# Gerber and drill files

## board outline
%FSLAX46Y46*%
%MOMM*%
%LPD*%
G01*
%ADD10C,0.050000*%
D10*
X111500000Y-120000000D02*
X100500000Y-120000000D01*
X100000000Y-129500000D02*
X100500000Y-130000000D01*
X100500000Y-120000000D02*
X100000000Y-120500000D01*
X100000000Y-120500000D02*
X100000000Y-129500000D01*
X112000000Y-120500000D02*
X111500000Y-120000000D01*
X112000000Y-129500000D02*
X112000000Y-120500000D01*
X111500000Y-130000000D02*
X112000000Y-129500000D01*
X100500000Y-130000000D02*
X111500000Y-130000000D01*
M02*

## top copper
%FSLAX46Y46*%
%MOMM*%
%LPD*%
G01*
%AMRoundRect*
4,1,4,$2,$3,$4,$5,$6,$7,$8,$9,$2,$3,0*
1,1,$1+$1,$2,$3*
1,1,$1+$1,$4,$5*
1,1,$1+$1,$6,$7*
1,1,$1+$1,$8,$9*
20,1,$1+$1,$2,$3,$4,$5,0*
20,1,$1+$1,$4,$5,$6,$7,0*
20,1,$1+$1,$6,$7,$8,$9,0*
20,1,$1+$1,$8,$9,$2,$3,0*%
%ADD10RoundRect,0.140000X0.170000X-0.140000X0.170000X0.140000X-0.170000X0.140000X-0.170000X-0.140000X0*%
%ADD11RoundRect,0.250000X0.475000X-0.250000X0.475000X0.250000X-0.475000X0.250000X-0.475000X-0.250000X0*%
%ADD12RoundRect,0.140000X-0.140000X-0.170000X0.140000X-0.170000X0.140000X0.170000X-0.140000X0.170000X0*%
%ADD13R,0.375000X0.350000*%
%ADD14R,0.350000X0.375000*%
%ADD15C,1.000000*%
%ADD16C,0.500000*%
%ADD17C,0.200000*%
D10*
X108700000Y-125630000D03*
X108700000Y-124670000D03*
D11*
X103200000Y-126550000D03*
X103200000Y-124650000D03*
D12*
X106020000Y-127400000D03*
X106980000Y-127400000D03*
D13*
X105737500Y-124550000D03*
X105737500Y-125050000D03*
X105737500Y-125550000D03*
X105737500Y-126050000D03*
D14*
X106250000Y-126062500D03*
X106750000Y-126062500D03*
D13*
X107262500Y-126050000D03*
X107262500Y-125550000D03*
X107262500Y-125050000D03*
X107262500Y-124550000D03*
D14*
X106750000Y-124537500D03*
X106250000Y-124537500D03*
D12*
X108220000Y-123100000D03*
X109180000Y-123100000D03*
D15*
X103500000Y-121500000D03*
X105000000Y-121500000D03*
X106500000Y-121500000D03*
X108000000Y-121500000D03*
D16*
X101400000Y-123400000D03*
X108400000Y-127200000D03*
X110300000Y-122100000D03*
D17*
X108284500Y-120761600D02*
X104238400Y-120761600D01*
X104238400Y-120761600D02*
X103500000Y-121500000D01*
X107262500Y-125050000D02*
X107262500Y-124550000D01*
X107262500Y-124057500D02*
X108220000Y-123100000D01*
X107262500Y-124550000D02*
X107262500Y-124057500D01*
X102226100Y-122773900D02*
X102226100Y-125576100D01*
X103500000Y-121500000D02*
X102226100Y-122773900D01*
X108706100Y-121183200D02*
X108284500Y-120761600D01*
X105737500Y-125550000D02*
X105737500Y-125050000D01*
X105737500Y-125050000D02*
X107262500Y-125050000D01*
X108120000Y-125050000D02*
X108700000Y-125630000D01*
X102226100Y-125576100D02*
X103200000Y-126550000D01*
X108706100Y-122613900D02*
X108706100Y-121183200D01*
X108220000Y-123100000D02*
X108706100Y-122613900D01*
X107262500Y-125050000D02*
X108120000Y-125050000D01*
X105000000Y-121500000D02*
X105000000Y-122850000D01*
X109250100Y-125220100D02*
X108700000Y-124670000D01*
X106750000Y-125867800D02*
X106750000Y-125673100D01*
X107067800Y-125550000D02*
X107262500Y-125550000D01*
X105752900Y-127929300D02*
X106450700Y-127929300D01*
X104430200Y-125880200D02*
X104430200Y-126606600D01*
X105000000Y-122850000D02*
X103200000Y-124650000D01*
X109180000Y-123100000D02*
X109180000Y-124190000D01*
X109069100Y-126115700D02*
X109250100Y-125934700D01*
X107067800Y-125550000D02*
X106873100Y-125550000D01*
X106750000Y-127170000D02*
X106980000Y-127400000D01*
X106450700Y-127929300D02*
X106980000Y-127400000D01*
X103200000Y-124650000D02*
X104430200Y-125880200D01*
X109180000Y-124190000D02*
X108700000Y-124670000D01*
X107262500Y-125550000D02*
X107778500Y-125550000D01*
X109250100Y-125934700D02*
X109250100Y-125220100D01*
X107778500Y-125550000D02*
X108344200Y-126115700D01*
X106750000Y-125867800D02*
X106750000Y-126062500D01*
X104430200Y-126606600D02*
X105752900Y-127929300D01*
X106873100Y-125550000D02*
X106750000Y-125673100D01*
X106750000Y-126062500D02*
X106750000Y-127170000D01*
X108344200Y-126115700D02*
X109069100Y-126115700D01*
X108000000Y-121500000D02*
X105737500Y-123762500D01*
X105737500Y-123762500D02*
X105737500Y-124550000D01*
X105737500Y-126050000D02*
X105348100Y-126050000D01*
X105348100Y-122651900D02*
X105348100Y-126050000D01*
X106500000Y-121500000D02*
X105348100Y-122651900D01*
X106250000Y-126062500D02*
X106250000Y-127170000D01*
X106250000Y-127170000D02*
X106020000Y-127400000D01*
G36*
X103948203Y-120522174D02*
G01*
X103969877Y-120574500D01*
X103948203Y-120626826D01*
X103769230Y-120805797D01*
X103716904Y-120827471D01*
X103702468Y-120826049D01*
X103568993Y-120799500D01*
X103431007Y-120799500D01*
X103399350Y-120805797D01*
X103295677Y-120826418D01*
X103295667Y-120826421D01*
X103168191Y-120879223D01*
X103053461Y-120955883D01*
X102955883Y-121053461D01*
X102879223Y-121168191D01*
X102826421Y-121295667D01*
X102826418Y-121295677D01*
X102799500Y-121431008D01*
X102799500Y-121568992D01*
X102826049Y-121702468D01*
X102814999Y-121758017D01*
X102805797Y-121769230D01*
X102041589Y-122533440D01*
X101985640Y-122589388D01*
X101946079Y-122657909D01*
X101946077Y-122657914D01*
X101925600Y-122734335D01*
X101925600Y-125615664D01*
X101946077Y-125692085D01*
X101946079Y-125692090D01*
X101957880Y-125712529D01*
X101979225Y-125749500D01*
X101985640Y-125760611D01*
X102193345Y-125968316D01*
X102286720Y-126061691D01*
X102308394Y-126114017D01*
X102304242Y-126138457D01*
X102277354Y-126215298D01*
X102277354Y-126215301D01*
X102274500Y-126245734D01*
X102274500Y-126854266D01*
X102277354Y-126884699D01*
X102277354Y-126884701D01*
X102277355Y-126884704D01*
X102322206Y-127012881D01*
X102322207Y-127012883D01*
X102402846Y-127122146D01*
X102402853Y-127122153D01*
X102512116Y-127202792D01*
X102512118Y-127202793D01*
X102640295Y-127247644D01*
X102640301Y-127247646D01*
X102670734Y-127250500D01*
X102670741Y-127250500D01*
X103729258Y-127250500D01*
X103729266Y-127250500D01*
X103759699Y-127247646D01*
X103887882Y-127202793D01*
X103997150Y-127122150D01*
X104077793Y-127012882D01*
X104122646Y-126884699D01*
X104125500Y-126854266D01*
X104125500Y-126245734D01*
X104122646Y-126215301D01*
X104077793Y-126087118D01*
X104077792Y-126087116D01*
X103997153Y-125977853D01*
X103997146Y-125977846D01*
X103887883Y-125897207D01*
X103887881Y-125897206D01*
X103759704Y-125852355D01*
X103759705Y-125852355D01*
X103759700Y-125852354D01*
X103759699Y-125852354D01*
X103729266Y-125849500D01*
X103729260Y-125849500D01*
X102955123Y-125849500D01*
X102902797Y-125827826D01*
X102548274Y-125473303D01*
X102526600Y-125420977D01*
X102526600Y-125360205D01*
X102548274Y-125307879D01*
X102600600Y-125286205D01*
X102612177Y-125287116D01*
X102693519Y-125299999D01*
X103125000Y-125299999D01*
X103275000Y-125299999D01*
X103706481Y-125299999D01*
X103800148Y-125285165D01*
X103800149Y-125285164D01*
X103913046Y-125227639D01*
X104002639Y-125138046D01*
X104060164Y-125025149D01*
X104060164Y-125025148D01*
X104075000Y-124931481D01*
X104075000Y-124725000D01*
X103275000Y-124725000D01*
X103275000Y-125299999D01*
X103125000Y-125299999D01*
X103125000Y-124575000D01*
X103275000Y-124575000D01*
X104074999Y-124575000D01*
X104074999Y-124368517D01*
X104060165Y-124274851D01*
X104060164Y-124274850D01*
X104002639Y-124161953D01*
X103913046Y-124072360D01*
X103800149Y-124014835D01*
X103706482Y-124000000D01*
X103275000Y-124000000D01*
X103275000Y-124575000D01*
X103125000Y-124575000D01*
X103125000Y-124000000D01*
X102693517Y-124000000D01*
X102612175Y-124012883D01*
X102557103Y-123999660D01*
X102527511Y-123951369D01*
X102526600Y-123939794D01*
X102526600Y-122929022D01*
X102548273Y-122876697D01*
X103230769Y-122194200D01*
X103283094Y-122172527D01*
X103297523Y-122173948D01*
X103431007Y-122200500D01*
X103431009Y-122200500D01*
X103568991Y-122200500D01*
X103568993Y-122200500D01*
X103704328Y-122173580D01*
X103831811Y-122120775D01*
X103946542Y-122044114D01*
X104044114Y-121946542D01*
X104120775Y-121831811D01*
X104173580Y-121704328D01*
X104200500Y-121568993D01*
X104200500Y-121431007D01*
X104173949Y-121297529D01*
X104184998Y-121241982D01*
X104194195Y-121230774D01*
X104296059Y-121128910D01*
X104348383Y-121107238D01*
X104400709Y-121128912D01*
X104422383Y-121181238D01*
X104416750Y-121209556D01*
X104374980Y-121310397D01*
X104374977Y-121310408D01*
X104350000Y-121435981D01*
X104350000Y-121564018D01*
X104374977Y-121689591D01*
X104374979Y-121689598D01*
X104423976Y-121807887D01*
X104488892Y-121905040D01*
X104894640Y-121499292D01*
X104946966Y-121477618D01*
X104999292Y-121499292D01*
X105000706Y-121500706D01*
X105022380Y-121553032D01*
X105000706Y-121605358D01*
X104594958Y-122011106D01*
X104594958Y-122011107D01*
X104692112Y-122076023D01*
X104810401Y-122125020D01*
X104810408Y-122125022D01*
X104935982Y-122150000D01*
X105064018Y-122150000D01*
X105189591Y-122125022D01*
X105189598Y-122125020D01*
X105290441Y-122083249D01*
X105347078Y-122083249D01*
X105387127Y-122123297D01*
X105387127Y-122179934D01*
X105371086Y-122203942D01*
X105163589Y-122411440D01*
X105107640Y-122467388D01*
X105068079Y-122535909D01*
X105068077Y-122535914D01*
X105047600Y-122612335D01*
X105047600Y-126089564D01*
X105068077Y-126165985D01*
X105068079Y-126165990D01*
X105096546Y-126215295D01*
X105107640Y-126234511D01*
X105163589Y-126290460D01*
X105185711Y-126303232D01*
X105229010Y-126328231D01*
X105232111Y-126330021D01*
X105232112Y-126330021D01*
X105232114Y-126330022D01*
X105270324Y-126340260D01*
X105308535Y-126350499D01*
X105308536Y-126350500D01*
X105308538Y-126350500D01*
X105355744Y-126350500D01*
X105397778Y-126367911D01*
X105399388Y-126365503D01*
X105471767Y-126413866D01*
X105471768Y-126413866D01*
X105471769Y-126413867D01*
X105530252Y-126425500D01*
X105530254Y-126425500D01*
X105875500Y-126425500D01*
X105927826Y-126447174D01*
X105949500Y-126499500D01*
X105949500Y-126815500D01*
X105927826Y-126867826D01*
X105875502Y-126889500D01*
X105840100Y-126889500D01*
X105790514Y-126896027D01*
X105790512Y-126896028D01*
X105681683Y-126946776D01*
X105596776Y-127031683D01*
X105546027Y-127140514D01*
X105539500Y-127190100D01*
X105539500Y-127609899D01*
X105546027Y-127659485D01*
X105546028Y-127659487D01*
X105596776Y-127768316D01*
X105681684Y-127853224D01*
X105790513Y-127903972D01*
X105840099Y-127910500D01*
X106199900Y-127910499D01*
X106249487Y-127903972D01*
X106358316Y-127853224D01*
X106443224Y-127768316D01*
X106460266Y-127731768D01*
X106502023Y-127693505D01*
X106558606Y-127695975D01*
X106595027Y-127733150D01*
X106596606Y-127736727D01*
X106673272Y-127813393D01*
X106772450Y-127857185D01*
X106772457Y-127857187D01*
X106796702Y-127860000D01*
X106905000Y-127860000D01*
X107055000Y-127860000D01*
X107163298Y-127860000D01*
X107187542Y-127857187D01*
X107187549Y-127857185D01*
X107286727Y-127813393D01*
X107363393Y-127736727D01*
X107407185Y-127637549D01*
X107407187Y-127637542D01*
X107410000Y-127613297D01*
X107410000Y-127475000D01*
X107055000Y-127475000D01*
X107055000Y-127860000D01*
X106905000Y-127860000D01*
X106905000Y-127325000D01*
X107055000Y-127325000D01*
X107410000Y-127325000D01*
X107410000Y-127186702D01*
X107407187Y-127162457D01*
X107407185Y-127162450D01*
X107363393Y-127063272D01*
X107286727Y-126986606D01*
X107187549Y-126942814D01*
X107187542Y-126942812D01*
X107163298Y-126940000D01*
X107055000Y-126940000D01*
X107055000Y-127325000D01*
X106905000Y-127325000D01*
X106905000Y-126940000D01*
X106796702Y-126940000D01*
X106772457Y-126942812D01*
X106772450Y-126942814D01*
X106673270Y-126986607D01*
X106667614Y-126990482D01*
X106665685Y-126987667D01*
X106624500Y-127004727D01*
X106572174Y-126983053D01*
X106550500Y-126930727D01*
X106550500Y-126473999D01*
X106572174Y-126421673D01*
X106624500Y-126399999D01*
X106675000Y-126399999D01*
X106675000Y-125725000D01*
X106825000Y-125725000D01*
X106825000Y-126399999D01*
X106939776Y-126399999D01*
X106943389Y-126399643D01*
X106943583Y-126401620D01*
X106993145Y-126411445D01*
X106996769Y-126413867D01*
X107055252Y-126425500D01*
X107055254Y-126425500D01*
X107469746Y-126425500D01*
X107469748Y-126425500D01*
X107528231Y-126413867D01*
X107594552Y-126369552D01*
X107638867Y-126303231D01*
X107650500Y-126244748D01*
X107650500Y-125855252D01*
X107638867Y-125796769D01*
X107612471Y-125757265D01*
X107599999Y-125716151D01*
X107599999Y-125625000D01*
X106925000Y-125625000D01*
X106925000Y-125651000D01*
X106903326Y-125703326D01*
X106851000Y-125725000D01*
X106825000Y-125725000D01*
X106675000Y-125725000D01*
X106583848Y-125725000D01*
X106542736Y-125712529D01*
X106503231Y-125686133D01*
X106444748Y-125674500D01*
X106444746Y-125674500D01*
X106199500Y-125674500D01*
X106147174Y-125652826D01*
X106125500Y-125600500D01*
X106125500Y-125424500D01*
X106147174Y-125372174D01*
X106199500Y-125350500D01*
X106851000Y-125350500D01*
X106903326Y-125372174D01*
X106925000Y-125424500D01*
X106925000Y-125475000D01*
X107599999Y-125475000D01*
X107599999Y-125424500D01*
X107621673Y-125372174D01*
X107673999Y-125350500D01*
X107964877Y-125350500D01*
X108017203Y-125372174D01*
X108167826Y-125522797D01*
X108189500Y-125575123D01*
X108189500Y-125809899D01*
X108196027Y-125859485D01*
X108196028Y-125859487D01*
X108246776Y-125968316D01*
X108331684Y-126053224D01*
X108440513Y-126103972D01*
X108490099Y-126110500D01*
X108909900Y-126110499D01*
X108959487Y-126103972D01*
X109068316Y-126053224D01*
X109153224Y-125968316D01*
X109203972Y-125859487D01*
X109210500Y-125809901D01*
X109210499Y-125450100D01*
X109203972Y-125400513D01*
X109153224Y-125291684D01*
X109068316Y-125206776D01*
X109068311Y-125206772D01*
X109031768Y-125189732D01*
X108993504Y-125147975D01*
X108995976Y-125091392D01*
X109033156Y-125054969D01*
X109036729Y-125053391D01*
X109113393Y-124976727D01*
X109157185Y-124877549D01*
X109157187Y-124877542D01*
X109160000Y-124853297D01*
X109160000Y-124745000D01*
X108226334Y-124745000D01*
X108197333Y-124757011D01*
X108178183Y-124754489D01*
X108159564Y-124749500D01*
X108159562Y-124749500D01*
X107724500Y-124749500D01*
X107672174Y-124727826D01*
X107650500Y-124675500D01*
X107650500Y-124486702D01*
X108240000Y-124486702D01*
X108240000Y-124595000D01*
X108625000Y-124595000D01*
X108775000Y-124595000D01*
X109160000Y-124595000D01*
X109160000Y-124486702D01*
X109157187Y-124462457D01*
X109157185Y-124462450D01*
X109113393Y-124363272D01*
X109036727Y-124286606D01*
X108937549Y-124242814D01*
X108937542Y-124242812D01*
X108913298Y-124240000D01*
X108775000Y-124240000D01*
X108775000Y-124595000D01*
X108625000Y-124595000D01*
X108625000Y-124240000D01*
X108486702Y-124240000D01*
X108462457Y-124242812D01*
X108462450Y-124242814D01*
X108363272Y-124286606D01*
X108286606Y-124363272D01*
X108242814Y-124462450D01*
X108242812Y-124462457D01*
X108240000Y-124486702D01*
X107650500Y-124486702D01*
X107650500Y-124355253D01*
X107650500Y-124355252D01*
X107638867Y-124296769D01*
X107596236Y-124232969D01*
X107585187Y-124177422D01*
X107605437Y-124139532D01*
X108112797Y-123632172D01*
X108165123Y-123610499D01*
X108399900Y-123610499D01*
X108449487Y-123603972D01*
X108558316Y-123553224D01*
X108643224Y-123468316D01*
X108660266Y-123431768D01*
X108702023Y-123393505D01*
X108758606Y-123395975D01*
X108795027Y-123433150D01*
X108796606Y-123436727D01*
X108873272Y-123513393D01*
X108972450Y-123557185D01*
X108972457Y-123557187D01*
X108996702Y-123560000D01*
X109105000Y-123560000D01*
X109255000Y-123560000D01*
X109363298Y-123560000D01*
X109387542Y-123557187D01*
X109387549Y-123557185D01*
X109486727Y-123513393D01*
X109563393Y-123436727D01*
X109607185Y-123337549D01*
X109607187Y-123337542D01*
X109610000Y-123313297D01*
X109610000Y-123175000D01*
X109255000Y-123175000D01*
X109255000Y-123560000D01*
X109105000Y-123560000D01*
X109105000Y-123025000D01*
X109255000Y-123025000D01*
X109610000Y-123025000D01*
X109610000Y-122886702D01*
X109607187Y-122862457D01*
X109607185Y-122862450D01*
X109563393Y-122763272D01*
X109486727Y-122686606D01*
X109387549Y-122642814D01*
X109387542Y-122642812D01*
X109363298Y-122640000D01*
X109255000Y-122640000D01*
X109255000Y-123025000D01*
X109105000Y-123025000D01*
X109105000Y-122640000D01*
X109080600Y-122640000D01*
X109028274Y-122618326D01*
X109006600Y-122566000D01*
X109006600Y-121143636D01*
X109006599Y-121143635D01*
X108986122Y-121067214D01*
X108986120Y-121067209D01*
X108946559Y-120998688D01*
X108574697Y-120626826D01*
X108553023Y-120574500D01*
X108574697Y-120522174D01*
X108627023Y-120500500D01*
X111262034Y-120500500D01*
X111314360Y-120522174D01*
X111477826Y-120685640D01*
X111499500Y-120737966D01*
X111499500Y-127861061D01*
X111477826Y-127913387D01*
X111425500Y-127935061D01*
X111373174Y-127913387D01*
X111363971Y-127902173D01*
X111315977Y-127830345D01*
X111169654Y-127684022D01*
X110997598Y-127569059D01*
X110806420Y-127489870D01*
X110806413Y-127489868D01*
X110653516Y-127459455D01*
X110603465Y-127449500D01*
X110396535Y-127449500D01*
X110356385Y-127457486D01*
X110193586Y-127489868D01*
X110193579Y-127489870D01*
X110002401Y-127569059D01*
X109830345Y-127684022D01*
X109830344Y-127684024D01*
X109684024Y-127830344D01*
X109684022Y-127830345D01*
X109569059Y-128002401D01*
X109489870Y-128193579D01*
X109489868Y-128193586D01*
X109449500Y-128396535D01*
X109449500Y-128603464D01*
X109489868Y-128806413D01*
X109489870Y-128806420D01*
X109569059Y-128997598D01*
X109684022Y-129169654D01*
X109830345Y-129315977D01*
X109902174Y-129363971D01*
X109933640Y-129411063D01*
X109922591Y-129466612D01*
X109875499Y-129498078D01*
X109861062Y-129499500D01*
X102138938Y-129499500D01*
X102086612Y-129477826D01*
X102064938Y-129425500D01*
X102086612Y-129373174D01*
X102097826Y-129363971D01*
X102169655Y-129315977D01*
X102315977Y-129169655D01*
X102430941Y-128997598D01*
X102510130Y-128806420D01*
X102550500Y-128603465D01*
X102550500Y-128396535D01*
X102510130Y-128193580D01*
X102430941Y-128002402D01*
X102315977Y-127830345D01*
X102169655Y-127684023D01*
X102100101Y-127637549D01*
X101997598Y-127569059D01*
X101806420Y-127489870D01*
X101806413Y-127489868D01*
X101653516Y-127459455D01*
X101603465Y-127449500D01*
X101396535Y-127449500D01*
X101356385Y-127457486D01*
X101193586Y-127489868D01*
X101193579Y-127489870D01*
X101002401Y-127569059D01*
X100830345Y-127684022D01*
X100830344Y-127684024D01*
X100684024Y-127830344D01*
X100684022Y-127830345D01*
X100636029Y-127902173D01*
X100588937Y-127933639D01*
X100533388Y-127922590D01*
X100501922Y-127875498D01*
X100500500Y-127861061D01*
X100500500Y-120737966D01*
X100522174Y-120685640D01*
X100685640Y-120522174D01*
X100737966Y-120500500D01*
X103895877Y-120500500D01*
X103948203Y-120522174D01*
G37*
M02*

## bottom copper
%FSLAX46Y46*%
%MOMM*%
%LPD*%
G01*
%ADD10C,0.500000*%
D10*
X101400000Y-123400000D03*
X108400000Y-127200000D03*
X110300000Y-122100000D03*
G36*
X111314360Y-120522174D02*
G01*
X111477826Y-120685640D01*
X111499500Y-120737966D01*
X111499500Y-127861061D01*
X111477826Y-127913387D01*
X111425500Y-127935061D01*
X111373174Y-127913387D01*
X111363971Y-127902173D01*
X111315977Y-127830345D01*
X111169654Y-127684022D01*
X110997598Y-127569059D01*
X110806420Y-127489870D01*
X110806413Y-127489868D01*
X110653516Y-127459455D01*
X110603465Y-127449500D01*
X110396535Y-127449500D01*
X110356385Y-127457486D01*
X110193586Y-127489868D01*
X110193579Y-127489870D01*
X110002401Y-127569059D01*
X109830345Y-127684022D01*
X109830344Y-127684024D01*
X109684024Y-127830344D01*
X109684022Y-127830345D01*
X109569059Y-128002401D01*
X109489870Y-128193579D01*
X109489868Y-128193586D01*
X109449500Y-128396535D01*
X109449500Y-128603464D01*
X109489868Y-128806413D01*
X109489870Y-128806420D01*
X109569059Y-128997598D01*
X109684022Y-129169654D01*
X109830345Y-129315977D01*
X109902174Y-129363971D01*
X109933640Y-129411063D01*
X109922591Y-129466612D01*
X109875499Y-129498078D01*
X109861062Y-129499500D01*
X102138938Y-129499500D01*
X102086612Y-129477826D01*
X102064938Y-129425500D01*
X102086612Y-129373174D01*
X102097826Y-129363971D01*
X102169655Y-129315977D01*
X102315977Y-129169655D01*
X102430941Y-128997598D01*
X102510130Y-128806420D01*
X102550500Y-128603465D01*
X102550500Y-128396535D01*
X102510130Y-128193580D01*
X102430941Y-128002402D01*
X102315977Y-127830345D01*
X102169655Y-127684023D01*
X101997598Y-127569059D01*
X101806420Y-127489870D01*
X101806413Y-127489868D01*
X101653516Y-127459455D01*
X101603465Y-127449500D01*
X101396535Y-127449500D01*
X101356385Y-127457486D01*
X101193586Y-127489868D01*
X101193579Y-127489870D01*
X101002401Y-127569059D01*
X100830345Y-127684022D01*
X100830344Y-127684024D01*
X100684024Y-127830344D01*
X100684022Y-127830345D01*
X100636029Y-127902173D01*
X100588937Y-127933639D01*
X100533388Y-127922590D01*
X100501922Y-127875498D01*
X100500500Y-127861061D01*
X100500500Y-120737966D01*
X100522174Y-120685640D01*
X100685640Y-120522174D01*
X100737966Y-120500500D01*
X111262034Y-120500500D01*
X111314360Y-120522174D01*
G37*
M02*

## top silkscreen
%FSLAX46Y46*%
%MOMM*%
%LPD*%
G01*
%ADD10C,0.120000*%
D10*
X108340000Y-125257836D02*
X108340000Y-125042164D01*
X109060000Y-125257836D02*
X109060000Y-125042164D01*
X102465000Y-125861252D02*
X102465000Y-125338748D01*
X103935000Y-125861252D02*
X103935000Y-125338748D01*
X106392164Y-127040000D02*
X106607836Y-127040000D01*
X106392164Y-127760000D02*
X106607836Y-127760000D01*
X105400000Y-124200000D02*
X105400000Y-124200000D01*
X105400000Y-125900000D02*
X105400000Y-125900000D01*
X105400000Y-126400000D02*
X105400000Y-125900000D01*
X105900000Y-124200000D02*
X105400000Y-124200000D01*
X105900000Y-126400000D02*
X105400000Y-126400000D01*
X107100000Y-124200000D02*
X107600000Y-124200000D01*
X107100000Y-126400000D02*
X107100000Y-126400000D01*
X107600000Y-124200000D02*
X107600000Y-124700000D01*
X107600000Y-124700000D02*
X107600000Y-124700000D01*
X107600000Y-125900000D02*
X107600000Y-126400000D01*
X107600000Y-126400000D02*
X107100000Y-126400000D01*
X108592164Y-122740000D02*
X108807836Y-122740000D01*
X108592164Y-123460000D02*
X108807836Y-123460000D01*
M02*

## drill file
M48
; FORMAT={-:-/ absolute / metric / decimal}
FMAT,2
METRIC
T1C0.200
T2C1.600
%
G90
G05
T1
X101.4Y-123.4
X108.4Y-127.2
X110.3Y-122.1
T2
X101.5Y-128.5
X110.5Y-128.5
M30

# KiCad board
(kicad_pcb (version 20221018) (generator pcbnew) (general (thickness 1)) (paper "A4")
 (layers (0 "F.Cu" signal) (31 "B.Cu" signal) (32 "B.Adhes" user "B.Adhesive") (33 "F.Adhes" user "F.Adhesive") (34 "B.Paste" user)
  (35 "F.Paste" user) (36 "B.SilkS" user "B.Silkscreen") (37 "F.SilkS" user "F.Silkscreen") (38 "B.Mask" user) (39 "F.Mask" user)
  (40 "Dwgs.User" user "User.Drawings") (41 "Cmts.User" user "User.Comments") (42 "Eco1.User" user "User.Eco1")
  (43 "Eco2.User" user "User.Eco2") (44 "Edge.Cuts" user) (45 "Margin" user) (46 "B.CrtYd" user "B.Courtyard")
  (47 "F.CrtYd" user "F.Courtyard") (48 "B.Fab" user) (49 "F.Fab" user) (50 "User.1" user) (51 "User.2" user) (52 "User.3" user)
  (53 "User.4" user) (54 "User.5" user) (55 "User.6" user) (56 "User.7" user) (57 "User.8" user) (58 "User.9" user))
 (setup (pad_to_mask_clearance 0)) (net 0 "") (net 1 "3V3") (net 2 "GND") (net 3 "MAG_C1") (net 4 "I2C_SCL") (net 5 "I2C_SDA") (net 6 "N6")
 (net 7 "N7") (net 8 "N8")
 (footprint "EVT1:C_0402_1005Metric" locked (layer "F.Cu") (at 108.7 125.15 90)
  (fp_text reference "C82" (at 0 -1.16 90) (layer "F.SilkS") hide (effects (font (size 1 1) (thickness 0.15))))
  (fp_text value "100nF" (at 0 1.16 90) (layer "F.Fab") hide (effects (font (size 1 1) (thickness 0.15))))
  (fp_line (start -0.107836 -0.36) (end 0.107836 -0.36) (stroke (width 0.12) (type solid)) (layer "F.SilkS"))
  (fp_line (start -0.107836 0.36) (end 0.107836 0.36) (stroke (width 0.12) (type solid)) (layer "F.SilkS"))
  (pad "1" smd roundrect locked (at -0.48 0 90) (size 0.56 0.62) (layers "F.Cu" "F.Paste" "F.Mask") (roundrect_rratio 0.25) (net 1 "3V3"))
  (pad "2" smd roundrect locked (at 0.48 0 90) (size 0.56 0.62) (layers "F.Cu" "F.Paste" "F.Mask") (roundrect_rratio 0.25) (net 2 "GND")))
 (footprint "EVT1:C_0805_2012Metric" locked (layer "F.Cu") (at 103.2 125.6 90)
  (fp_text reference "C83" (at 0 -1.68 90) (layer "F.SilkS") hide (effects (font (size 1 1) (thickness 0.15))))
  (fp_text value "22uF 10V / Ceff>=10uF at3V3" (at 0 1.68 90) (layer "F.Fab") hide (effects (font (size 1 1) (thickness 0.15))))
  (fp_line (start -0.261252 -0.735) (end 0.261252 -0.735) (stroke (width 0.12) (type solid)) (layer "F.SilkS"))
  (fp_line (start -0.261252 0.735) (end 0.261252 0.735) (stroke (width 0.12) (type solid)) (layer "F.SilkS"))
  (pad "1" smd roundrect locked (at -0.95 0 90) (size 1 1.45) (layers "F.Cu" "F.Paste" "F.Mask") (roundrect_rratio 0.25) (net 1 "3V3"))
  (pad "2" smd roundrect locked (at 0.95 0 90) (size 1 1.45) (layers "F.Cu" "F.Paste" "F.Mask") (roundrect_rratio 0.25) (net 2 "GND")))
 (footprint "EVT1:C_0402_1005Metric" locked (layer "F.Cu") (at 106.5 127.4)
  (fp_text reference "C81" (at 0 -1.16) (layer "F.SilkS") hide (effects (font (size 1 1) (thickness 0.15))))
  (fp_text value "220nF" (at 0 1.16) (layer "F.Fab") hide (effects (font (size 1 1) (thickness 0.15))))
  (fp_line (start -0.107836 -0.36) (end 0.107836 -0.36) (stroke (width 0.12) (type solid)) (layer "F.SilkS"))
  (fp_line (start -0.107836 0.36) (end 0.107836 0.36) (stroke (width 0.12) (type solid)) (layer "F.SilkS"))
  (pad "1" smd roundrect locked (at -0.48 0) (size 0.56 0.62) (layers "F.Cu" "F.Paste" "F.Mask") (roundrect_rratio 0.25) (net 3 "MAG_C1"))
  (pad "2" smd roundrect locked (at 0.48 0) (size 0.56 0.62) (layers "F.Cu" "F.Paste" "F.Mask") (roundrect_rratio 0.25) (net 2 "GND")))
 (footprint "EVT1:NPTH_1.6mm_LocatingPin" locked (layer "F.Cu") (at 101.5 128.5)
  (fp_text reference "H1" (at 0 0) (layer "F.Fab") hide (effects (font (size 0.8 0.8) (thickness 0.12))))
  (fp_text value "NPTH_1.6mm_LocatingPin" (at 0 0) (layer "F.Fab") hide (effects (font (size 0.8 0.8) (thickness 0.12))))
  (pad "" np_thru_hole circle locked (at 0 0) (size 1.6 1.6) (drill 1.6) (layers "*.Cu" "*.Mask")))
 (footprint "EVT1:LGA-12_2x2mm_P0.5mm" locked (layer "F.Cu") (at 106.5 125.3)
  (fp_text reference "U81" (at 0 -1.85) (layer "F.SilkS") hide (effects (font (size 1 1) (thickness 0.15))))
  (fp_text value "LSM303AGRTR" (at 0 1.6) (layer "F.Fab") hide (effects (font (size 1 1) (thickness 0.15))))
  (fp_line (start -1.1 -1.1) (end -1.1 -1.1) (stroke (width 0.12) (type solid)) (layer "F.SilkS"))
  (fp_line (start -1.1 0.6) (end -1.1 0.6) (stroke (width 0.12) (type solid)) (layer "F.SilkS"))
  (fp_line (start -1.1 1.1) (end -1.1 0.6) (stroke (width 0.12) (type solid)) (layer "F.SilkS"))
  (fp_line (start -0.6 -1.1) (end -1.1 -1.1) (stroke (width 0.12) (type solid)) (layer "F.SilkS"))
  (fp_line (start -0.6 1.1) (end -1.1 1.1) (stroke (width 0.12) (type solid)) (layer "F.SilkS"))
  (fp_line (start 0.6 -1.1) (end 1.1 -1.1) (stroke (width 0.12) (type solid)) (layer "F.SilkS"))
  (fp_line (start 0.6 1.1) (end 0.6 1.1) (stroke (width 0.12) (type solid)) (layer "F.SilkS"))
  (fp_line (start 1.1 -1.1) (end 1.1 -0.6) (stroke (width 0.12) (type solid)) (layer "F.SilkS"))
  (fp_line (start 1.1 -0.6) (end 1.1 -0.6) (stroke (width 0.12) (type solid)) (layer "F.SilkS"))
  (fp_line (start 1.1 0.6) (end 1.1 1.1) (stroke (width 0.12) (type solid)) (layer "F.SilkS"))
  (fp_line (start 1.1 1.1) (end 0.6 1.1) (stroke (width 0.12) (type solid)) (layer "F.SilkS"))
  (pad "1" smd rect locked (at -0.7625 -0.75) (size 0.375 0.35) (layers "F.Cu" "F.Paste" "F.Mask") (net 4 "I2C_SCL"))
  (pad "2" smd rect locked (at -0.7625 -0.25) (size 0.375 0.35) (layers "F.Cu" "F.Paste" "F.Mask") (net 1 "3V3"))
  (pad "3" smd rect locked (at -0.7625 0.25) (size 0.375 0.35) (layers "F.Cu" "F.Paste" "F.Mask") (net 1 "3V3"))
  (pad "4" smd rect locked (at -0.7625 0.75) (size 0.375 0.35) (layers "F.Cu" "F.Paste" "F.Mask") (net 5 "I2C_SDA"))
  (pad "5" smd rect locked (at -0.25 0.7625 90) (size 0.375 0.35) (layers "F.Cu" "F.Paste" "F.Mask") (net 3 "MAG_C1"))
  (pad "6" smd rect locked (at 0.25 0.7625 90) (size 0.375 0.35) (layers "F.Cu" "F.Paste" "F.Mask") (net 2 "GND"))
  (pad "7" smd rect locked (at 0.7625 0.75) (size 0.375 0.35) (layers "F.Cu" "F.Paste" "F.Mask") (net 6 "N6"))
  (pad "8" smd rect locked (at 0.7625 0.25) (size 0.375 0.35) (layers "F.Cu" "F.Paste" "F.Mask") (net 2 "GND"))
  (pad "9" smd rect locked (at 0.7625 -0.25) (size 0.375 0.35) (layers "F.Cu" "F.Paste" "F.Mask") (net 1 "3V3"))
  (pad "10" smd rect locked (at 0.7625 -0.75) (size 0.375 0.35) (layers "F.Cu" "F.Paste" "F.Mask") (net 1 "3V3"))
  (pad "11" smd rect locked (at 0.25 -0.7625 90) (size 0.375 0.35) (layers "F.Cu" "F.Paste" "F.Mask") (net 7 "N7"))
  (pad "12" smd rect locked (at -0.25 -0.7625 90) (size 0.375 0.35) (layers "F.Cu" "F.Paste" "F.Mask") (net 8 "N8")))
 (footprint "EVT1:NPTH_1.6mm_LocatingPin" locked (layer "F.Cu") (at 110.5 128.5)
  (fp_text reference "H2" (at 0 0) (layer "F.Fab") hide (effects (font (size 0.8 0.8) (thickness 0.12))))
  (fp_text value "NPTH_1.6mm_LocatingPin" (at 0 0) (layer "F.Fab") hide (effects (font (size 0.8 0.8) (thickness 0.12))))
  (pad "" np_thru_hole circle locked (at 0 0) (size 1.6 1.6) (drill 1.6) (layers "*.Cu" "*.Mask")))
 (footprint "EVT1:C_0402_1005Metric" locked (layer "F.Cu") (at 108.7 123.1)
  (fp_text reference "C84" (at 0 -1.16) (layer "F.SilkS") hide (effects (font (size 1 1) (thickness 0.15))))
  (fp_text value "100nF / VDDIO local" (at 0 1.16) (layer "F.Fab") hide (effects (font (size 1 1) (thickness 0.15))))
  (fp_line (start -0.107836 -0.36) (end 0.107836 -0.36) (stroke (width 0.12) (type solid)) (layer "F.SilkS"))
  (fp_line (start -0.107836 0.36) (end 0.107836 0.36) (stroke (width 0.12) (type solid)) (layer "F.SilkS"))
  (pad "1" smd roundrect locked (at -0.48 0) (size 0.56 0.62) (layers "F.Cu" "F.Paste" "F.Mask") (roundrect_rratio 0.25) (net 1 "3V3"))
  (pad "2" smd roundrect locked (at 0.48 0) (size 0.56 0.62) (layers "F.Cu" "F.Paste" "F.Mask") (roundrect_rratio 0.25) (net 2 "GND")))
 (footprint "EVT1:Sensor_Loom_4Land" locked (layer "F.Cu") (at 103.5 121.5)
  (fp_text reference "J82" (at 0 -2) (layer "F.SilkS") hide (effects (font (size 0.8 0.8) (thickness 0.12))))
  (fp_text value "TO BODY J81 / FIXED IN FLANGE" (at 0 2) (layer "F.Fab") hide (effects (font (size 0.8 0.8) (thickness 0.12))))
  (pad "1" smd circle locked (at 0 0) (size 1 1) (layers "F.Cu" "F.Paste" "F.Mask") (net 1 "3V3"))
  (pad "2" smd circle locked (at 1.5 0) (size 1 1) (layers "F.Cu" "F.Paste" "F.Mask") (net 2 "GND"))
  (pad "3" smd circle locked (at 3 0) (size 1 1) (layers "F.Cu" "F.Paste" "F.Mask") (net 5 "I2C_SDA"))
  (pad "4" smd circle locked (at 4.5 0) (size 1 1) (layers "F.Cu" "F.Paste" "F.Mask") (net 4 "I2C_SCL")))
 (gr_line (start 111.5 120) (end 100.5 120) (stroke (width 0.05) (type default)) (layer "Edge.Cuts"))
 (gr_line (start 100 129.5) (end 100.5 130) (stroke (width 0.05) (type default)) (layer "Edge.Cuts"))
 (gr_line (start 100.5 120) (end 100 120.5) (stroke (width 0.05) (type default)) (layer "Edge.Cuts"))
 (gr_line (start 100 120.5) (end 100 129.5) (stroke (width 0.05) (type default)) (layer "Edge.Cuts"))
 (gr_line (start 112 120.5) (end 111.5 120) (stroke (width 0.05) (type default)) (layer "Edge.Cuts"))
 (gr_line (start 112 129.5) (end 112 120.5) (stroke (width 0.05) (type default)) (layer "Edge.Cuts"))
 (gr_line (start 111.5 130) (end 112 129.5) (stroke (width 0.05) (type default)) (layer "Edge.Cuts"))
 (gr_line (start 100.5 130) (end 111.5 130) (stroke (width 0.05) (type default)) (layer "Edge.Cuts"))
 (segment (start 108.2845 120.7616) (end 104.2384 120.7616) (width 0.2) (layer "F.Cu") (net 1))
 (segment (start 104.2384 120.7616) (end 103.5 121.5) (width 0.2) (layer "F.Cu") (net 1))
 (segment (start 107.2625 125.05) (end 107.2625 124.55) (width 0.2) (layer "F.Cu") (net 1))
 (segment (start 107.2625 124.0575) (end 108.22 123.1) (width 0.2) (layer "F.Cu") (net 1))
 (segment (start 107.2625 124.55) (end 107.2625 124.0575) (width 0.2) (layer "F.Cu") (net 1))
 (segment (start 102.2261 122.7739) (end 102.2261 125.5761) (width 0.2) (layer "F.Cu") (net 1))
 (segment (start 103.5 121.5) (end 102.2261 122.7739) (width 0.2) (layer "F.Cu") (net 1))
 (segment (start 108.7061 121.1832) (end 108.2845 120.7616) (width 0.2) (layer "F.Cu") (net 1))
 (segment (start 105.7375 125.55) (end 105.7375 125.05) (width 0.2) (layer "F.Cu") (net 1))
 (segment (start 105.7375 125.05) (end 107.2625 125.05) (width 0.2) (layer "F.Cu") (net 1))
 (segment (start 108.12 125.05) (end 108.7 125.63) (width 0.2) (layer "F.Cu") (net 1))
 (segment (start 102.2261 125.5761) (end 103.2 126.55) (width 0.2) (layer "F.Cu") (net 1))
 (segment (start 108.7061 122.6139) (end 108.7061 121.1832) (width 0.2) (layer "F.Cu") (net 1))
 (segment (start 108.22 123.1) (end 108.7061 122.6139) (width 0.2) (layer "F.Cu") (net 1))
 (segment (start 107.2625 125.05) (end 108.12 125.05) (width 0.2) (layer "F.Cu") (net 1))
 (segment (start 105 121.5) (end 105 122.85) (width 0.2) (layer "F.Cu") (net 2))
 (segment (start 109.2501 125.2201) (end 108.7 124.67) (width 0.2) (layer "F.Cu") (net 2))
 (segment (start 106.75 125.8678) (end 106.75 125.6731) (width 0.2) (layer "F.Cu") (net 2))
 (segment (start 107.0678 125.55) (end 107.2625 125.55) (width 0.2) (layer "F.Cu") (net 2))
 (segment (start 105.7529 127.9293) (end 106.4507 127.9293) (width 0.2) (layer "F.Cu") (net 2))
 (segment (start 104.4302 125.8802) (end 104.4302 126.6066) (width 0.2) (layer "F.Cu") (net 2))
 (segment (start 105 122.85) (end 103.2 124.65) (width 0.2) (layer "F.Cu") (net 2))
 (segment (start 109.18 123.1) (end 109.18 124.19) (width 0.2) (layer "F.Cu") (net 2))
 (segment (start 109.0691 126.1157) (end 109.2501 125.9347) (width 0.2) (layer "F.Cu") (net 2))
 (segment (start 107.0678 125.55) (end 106.8731 125.55) (width 0.2) (layer "F.Cu") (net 2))
 (segment (start 106.75 127.17) (end 106.98 127.4) (width 0.2) (layer "F.Cu") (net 2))
 (segment (start 106.4507 127.9293) (end 106.98 127.4) (width 0.2) (layer "F.Cu") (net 2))
 (segment (start 103.2 124.65) (end 104.4302 125.8802) (width 0.2) (layer "F.Cu") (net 2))
 (segment (start 109.18 124.19) (end 108.7 124.67) (width 0.2) (layer "F.Cu") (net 2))
 (segment (start 107.2625 125.55) (end 107.7785 125.55) (width 0.2) (layer "F.Cu") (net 2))
 (segment (start 109.2501 125.9347) (end 109.2501 125.2201) (width 0.2) (layer "F.Cu") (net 2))
 (segment (start 107.7785 125.55) (end 108.3442 126.1157) (width 0.2) (layer "F.Cu") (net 2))
 (segment (start 106.75 125.8678) (end 106.75 126.0625) (width 0.2) (layer "F.Cu") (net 2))
 (segment (start 104.4302 126.6066) (end 105.7529 127.9293) (width 0.2) (layer "F.Cu") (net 2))
 (segment (start 106.8731 125.55) (end 106.75 125.6731) (width 0.2) (layer "F.Cu") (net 2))
 (segment (start 106.75 126.0625) (end 106.75 127.17) (width 0.2) (layer "F.Cu") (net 2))
 (segment (start 108.3442 126.1157) (end 109.0691 126.1157) (width 0.2) (layer "F.Cu") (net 2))
 (via (at 101.4 123.4) (size 0.5) (drill 0.2) (layers "F.Cu" "B.Cu") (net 2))
 (via (at 108.4 127.2) (size 0.5) (drill 0.2) (layers "F.Cu" "B.Cu") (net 2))
 (via (at 110.3 122.1) (size 0.5) (drill 0.2) (layers "F.Cu" "B.Cu") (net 2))
 (segment (start 108 121.5) (end 105.7375 123.7625) (width 0.2) (layer "F.Cu") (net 4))
 (segment (start 105.7375 123.7625) (end 105.7375 124.55) (width 0.2) (layer "F.Cu") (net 4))
 (segment (start 105.7375 126.05) (end 105.3481 126.05) (width 0.2) (layer "F.Cu") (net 5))
 (segment (start 105.3481 122.6519) (end 105.3481 126.05) (width 0.2) (layer "F.Cu") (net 5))
 (segment (start 106.5 121.5) (end 105.3481 122.6519) (width 0.2) (layer "F.Cu") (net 5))
 (segment (start 106.25 126.0625) (end 106.25 127.17) (width 0.2) (layer "F.Cu") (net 3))
 (segment (start 106.25 127.17) (end 106.02 127.4) (width 0.2) (layer "F.Cu") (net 3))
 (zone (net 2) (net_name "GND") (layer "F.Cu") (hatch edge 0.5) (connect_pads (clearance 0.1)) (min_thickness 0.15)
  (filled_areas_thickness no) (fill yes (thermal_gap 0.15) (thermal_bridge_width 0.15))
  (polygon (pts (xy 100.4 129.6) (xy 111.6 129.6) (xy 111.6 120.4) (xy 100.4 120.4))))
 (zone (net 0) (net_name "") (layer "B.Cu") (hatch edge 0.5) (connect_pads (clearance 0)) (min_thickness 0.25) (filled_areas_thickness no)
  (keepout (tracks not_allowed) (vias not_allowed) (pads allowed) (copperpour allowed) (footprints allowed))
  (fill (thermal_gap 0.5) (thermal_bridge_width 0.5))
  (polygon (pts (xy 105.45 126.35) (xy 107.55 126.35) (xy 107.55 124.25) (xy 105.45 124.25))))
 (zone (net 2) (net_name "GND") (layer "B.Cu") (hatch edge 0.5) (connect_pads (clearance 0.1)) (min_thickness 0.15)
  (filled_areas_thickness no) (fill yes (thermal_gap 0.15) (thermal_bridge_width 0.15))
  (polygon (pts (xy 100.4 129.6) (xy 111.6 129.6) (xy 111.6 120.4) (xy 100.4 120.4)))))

